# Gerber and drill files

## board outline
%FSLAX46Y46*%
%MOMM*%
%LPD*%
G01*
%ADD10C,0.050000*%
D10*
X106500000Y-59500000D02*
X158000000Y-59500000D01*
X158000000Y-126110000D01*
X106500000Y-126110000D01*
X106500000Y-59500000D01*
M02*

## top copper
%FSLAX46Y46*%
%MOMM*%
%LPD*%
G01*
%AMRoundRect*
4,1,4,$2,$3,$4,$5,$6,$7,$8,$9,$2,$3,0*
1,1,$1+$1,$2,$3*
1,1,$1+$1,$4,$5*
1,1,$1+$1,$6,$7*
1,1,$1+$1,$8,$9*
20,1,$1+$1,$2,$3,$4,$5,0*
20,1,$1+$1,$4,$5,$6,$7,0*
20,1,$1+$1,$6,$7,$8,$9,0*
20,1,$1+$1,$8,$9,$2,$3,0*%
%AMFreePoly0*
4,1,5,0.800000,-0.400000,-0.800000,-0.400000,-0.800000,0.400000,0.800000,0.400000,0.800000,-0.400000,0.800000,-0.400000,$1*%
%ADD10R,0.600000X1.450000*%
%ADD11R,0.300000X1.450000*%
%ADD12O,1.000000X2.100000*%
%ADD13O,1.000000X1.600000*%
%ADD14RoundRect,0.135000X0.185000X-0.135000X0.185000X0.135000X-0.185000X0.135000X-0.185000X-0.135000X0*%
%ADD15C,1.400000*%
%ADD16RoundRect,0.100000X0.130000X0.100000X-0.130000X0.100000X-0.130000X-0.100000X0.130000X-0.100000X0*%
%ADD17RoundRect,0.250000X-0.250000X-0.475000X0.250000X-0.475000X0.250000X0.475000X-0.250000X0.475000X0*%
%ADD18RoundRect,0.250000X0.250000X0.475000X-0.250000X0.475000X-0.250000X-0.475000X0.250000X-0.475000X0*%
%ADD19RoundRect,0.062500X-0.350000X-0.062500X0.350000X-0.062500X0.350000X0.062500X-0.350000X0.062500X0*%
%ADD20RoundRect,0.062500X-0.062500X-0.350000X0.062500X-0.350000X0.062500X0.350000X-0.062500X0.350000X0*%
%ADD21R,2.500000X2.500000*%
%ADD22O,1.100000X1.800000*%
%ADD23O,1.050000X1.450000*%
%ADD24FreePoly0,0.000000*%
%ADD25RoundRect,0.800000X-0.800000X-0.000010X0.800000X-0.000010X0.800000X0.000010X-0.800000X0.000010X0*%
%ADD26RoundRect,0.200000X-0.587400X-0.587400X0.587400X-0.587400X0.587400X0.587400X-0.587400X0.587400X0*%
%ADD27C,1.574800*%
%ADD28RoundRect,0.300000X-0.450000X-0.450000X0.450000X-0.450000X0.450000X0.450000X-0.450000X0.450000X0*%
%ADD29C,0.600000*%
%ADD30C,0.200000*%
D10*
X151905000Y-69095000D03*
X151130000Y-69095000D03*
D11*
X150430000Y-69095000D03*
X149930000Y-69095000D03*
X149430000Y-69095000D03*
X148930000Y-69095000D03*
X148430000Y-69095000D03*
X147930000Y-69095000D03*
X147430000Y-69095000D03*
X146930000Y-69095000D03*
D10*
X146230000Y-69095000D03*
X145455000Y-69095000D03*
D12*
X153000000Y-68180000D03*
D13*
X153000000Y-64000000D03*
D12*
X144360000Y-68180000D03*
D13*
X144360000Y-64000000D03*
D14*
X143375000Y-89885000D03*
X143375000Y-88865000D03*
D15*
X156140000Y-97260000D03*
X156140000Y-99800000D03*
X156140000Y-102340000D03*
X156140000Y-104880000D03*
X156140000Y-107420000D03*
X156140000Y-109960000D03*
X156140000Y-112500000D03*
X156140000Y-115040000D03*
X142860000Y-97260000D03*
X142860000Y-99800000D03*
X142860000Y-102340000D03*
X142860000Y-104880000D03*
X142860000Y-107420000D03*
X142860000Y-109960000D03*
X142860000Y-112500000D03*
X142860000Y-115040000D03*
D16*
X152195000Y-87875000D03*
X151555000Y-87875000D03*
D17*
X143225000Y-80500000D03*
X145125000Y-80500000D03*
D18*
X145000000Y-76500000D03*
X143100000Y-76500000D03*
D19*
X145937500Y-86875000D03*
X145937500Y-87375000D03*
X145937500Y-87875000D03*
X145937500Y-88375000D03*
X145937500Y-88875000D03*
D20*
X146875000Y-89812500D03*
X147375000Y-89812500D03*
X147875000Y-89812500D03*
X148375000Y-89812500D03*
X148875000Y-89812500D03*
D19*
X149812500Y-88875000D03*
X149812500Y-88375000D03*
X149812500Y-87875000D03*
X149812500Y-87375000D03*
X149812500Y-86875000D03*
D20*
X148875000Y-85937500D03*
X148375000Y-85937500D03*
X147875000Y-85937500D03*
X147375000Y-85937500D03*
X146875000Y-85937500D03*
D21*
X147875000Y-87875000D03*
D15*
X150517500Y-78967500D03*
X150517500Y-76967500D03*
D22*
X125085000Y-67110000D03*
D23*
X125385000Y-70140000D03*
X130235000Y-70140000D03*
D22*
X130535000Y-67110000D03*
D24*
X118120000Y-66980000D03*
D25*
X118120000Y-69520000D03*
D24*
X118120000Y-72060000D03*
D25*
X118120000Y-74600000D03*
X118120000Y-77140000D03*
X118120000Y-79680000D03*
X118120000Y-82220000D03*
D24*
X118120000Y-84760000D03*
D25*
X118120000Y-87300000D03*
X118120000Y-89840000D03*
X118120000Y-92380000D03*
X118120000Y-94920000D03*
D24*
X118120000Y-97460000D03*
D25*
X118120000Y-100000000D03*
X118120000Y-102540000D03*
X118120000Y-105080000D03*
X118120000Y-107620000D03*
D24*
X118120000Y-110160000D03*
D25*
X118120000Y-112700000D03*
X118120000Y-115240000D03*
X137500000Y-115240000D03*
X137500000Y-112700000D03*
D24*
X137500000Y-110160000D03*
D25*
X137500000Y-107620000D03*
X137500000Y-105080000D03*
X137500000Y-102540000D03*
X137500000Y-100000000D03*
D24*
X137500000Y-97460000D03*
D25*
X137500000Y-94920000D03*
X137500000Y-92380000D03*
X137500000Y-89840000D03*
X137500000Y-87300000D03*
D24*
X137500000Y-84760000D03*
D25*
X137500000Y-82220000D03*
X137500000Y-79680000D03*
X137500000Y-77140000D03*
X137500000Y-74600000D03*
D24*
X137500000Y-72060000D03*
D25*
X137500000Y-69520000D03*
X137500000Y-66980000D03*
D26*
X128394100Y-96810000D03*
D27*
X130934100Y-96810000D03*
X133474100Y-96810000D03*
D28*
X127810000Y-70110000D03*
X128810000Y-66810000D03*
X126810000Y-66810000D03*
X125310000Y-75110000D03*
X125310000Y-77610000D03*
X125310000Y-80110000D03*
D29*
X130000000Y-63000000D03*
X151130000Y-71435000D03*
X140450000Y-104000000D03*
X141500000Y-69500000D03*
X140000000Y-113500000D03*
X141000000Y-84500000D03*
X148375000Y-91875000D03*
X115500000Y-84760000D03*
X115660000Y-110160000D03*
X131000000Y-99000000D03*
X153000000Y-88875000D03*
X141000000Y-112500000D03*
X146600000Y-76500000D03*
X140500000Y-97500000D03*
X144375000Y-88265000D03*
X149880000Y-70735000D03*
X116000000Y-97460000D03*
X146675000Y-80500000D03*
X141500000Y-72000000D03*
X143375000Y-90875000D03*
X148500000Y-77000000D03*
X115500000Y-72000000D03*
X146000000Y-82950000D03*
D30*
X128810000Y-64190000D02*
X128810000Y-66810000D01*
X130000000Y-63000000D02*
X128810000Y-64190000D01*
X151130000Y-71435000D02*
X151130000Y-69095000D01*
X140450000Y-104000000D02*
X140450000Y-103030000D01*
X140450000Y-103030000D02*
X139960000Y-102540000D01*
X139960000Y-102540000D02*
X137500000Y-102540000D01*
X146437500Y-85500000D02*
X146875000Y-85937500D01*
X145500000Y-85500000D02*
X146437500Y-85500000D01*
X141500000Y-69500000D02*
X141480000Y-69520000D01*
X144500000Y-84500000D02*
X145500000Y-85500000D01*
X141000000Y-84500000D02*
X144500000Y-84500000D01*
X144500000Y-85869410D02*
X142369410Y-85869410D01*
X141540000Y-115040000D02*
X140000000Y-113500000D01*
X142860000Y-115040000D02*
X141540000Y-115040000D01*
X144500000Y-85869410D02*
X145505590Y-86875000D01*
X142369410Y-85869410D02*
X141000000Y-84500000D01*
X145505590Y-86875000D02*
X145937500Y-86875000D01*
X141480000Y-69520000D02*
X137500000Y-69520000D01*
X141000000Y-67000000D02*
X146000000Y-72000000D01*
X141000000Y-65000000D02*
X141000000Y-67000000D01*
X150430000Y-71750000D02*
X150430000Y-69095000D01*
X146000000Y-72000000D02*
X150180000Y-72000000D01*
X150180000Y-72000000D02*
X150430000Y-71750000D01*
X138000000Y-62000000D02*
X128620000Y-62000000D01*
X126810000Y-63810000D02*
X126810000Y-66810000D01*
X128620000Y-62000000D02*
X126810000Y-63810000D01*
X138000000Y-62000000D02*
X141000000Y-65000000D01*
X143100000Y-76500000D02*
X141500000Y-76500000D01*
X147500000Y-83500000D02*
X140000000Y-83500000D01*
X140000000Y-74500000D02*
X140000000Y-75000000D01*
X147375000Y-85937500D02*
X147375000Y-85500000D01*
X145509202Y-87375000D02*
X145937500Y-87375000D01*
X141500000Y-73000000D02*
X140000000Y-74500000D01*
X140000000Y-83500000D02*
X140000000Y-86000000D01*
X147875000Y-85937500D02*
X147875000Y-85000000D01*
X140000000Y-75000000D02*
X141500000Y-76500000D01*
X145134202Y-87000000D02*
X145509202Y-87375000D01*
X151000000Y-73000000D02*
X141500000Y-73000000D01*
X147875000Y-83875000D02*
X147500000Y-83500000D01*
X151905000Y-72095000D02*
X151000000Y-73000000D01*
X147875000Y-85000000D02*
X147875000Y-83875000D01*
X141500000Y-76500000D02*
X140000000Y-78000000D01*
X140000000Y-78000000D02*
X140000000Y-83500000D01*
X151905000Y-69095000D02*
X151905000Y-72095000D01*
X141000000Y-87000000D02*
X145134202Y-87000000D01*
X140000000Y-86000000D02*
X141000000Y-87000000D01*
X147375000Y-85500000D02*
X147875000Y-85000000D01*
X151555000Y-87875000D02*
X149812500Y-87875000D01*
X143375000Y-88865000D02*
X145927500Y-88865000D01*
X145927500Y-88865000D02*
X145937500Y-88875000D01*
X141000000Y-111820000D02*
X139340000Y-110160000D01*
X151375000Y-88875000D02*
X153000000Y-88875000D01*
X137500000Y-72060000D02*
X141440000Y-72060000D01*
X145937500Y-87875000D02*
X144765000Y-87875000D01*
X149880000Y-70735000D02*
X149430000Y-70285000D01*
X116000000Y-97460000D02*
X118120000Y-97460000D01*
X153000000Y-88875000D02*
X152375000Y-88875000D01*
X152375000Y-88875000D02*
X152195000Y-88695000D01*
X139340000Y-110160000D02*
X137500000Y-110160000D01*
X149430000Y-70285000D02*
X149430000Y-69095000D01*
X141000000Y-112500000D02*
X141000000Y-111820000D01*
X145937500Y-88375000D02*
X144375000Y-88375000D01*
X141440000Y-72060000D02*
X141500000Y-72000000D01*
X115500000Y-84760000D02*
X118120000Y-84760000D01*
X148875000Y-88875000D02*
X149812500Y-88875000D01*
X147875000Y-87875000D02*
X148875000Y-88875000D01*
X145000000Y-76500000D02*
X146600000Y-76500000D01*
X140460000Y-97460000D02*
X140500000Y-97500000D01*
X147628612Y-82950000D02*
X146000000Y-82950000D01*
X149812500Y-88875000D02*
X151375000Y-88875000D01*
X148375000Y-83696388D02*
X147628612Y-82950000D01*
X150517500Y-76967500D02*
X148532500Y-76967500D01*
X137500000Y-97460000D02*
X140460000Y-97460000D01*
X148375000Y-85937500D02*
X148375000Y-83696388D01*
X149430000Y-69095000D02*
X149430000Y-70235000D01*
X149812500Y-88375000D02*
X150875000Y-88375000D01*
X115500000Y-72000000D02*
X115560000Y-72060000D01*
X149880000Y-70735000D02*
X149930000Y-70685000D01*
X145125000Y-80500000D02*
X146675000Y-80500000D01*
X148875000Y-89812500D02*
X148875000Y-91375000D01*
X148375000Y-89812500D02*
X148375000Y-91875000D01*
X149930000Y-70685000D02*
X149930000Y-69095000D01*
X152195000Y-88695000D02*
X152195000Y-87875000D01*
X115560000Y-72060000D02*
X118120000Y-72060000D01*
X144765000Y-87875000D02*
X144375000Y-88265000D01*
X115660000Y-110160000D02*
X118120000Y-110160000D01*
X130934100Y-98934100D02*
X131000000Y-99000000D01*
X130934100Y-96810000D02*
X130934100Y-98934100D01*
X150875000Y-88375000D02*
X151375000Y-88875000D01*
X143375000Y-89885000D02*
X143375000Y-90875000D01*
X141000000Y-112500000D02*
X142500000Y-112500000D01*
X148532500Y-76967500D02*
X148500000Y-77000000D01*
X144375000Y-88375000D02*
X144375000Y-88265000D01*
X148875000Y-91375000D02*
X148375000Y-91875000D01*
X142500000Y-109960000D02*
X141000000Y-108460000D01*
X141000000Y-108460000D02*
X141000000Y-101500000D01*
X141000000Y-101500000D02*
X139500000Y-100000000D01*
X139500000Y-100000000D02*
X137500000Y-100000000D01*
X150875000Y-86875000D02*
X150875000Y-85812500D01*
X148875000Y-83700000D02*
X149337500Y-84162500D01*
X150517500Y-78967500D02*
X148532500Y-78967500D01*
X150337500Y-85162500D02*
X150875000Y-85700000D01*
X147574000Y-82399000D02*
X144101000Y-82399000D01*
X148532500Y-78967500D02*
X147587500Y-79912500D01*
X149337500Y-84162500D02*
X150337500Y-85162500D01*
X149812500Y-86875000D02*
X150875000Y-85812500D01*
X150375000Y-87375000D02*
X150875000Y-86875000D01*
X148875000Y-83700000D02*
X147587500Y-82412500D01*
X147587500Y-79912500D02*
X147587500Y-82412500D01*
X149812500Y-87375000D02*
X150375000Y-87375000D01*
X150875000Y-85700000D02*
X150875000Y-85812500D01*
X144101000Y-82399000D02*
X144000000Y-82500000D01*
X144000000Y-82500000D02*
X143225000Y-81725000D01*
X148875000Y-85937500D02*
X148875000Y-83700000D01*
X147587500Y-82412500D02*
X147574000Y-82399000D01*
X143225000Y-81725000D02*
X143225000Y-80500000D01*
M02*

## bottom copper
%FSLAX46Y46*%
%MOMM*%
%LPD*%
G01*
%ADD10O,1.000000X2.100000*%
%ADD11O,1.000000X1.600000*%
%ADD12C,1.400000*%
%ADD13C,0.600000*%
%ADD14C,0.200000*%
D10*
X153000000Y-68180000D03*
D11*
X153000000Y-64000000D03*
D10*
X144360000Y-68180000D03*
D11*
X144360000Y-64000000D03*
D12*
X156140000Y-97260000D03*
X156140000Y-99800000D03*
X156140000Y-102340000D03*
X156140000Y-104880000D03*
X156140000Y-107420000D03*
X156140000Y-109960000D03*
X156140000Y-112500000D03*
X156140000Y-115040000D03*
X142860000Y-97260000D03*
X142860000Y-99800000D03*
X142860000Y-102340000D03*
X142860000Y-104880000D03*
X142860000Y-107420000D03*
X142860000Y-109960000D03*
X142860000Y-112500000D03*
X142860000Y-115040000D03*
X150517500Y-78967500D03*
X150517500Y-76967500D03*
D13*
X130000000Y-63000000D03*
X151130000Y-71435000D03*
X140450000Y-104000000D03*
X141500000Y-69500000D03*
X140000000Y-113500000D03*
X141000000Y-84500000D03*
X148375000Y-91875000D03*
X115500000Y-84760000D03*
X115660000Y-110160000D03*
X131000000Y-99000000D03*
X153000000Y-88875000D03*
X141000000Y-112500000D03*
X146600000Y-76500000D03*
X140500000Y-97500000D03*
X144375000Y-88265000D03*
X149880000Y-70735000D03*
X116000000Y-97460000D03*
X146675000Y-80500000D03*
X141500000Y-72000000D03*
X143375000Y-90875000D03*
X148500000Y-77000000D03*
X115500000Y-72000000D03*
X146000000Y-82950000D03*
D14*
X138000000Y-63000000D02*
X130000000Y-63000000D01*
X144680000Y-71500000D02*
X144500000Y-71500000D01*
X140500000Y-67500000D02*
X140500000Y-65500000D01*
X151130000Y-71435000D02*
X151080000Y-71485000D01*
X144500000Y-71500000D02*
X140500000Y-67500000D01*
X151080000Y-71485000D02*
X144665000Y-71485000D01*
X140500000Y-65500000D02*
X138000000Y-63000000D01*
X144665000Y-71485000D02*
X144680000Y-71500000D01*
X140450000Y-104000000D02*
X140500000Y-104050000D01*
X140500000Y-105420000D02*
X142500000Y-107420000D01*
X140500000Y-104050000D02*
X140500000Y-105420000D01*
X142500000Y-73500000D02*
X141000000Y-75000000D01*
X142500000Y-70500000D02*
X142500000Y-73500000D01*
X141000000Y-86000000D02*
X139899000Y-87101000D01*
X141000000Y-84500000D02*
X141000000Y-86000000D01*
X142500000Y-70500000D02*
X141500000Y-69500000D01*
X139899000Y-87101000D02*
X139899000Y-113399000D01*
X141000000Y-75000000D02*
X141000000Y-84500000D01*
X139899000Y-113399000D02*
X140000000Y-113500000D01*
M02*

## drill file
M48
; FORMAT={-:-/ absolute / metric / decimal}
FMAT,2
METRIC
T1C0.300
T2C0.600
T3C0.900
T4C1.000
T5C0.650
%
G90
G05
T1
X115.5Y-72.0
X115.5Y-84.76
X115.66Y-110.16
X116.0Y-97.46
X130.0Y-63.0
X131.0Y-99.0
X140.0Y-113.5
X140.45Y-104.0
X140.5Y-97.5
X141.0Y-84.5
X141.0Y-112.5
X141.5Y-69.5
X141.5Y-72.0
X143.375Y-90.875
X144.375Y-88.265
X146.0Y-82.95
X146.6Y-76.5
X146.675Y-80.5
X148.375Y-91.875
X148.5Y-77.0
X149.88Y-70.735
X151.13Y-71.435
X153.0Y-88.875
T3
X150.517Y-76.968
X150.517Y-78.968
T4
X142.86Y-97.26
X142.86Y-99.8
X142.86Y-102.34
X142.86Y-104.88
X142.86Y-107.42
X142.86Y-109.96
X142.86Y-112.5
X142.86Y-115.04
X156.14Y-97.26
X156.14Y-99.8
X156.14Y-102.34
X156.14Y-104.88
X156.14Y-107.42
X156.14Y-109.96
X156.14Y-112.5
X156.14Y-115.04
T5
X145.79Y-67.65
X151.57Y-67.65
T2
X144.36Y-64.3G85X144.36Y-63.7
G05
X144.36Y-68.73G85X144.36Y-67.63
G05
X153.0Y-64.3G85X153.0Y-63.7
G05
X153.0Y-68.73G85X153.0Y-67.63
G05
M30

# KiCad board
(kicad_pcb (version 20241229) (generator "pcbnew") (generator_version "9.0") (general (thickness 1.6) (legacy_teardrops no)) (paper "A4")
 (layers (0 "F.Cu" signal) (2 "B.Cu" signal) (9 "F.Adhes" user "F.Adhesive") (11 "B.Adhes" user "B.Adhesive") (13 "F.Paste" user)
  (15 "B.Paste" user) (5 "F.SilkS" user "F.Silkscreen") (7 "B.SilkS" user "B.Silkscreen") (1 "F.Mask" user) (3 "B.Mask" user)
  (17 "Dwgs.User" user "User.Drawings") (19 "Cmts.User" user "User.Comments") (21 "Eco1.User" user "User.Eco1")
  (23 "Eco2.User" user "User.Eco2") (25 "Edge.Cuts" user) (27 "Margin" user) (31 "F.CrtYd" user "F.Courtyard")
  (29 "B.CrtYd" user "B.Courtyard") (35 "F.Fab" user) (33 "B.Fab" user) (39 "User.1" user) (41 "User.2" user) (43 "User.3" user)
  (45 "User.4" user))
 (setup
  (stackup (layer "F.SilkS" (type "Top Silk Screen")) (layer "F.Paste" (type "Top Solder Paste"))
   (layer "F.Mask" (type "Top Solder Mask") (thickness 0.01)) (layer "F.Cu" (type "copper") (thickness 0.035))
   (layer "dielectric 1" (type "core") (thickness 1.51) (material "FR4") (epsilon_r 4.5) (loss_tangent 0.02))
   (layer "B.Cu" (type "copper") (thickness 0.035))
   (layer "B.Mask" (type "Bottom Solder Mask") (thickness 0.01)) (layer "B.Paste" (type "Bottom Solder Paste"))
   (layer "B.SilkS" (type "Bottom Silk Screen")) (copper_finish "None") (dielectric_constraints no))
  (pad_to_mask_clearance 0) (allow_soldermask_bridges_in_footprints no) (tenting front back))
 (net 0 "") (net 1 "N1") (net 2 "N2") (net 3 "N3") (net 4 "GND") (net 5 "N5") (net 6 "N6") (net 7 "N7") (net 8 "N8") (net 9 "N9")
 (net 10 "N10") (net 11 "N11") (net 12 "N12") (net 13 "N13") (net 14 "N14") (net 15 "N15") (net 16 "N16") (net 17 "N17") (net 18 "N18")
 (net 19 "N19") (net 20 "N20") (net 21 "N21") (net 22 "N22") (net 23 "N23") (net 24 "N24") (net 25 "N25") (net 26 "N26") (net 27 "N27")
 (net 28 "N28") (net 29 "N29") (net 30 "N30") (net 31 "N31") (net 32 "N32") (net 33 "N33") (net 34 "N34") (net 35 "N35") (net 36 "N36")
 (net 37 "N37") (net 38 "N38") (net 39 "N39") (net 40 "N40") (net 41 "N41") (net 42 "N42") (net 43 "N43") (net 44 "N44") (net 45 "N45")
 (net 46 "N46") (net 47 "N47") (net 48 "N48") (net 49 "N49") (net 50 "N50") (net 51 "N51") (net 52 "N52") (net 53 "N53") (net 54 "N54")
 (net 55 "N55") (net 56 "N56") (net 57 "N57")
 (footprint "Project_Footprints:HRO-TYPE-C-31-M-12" (layer "F.Cu") (at 148.68 61.4 180)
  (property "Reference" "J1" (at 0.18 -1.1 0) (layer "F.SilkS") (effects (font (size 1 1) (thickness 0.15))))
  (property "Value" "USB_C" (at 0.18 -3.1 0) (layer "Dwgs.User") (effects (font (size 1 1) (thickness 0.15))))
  (pad "" np_thru_hole circle (at -2.89 -6.25 180) (size 0.65 0.65) (drill 0.65) (layers "*.Cu" "*.Mask"))
  (pad "" np_thru_hole circle (at 2.89 -6.25 180) (size 0.65 0.65) (drill 0.65) (layers "*.Cu" "*.Mask"))
  (pad "1" smd rect (at -3.225 -7.695 180) (size 0.6 1.45) (layers "F.Cu" "F.Mask" "F.Paste") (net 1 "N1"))
  (pad "2" smd rect (at -2.45 -7.695 180) (size 0.6 1.45) (layers "F.Cu" "F.Mask" "F.Paste") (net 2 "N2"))
  (pad "3" smd rect (at -1.75 -7.695 180) (size 0.3 1.45) (layers "F.Cu" "F.Mask" "F.Paste") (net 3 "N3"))
  (pad "4" smd rect (at -1.25 -7.695 180) (size 0.3 1.45) (layers "F.Cu" "F.Mask" "F.Paste") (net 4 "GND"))
  (pad "5" smd rect (at -0.75 -7.695 180) (size 0.3 1.45) (layers "F.Cu" "F.Mask" "F.Paste") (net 4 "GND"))
  (pad "6" smd rect (at -0.25 -7.695 180) (size 0.3 1.45) (layers "F.Cu" "F.Mask" "F.Paste"))
  (pad "7" smd rect (at 0.25 -7.695 180) (size 0.3 1.45) (layers "F.Cu" "F.Mask" "F.Paste"))
  (pad "8" smd rect (at 0.75 -7.695 180) (size 0.3 1.45) (layers "F.Cu" "F.Mask" "F.Paste"))
  (pad "9" smd rect (at 1.25 -7.695 180) (size 0.3 1.45) (layers "F.Cu" "F.Mask" "F.Paste"))
  (pad "10" smd rect (at 1.75 -7.695 180) (size 0.3 1.45) (layers "F.Cu" "F.Mask" "F.Paste"))
  (pad "11" smd rect (at 2.45 -7.695 180) (size 0.6 1.45) (layers "F.Cu" "F.Mask" "F.Paste"))
  (pad "12" smd rect (at 3.225 -7.695 180) (size 0.6 1.45) (layers "F.Cu" "F.Mask" "F.Paste"))
  (pad "13" thru_hole oval (at -4.32 -6.78 180) (size 1 2.1) (drill oval 0.6 1.7) (layers "*.Cu" "B.Mask") (remove_unused_layers no))
  (pad "13" thru_hole oval (at -4.32 -2.6 180) (size 1 1.6) (drill oval 0.6 1.2) (layers "*.Cu" "B.Mask") (remove_unused_layers no))
  (pad "13" thru_hole oval (at 4.32 -6.78 180) (size 1 2.1) (drill oval 0.6 1.7) (layers "*.Cu" "B.Mask") (remove_unused_layers no))
  (pad "13" thru_hole oval (at 4.32 -2.6 180) (size 1 1.6) (drill oval 0.6 1.2) (layers "*.Cu" "B.Mask") (remove_unused_layers no)))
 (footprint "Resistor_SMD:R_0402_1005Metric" (layer "F.Cu") (at 143.375 89.375 90)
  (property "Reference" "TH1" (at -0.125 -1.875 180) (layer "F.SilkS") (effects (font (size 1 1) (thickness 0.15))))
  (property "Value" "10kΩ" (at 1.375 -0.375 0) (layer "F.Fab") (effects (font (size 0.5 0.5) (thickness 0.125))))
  (pad "1" smd roundrect (at -0.51 0 90) (size 0.54 0.64) (layers "F.Cu" "F.Mask" "F.Paste") (roundrect_rratio 0.25) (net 4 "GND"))
  (pad "2" smd roundrect (at 0.51 0 90) (size 0.54 0.64) (layers "F.Cu" "F.Mask" "F.Paste") (roundrect_rratio 0.25) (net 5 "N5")))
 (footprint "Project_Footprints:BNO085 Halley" (layer "F.Cu") (at 156.14 97.26 -90)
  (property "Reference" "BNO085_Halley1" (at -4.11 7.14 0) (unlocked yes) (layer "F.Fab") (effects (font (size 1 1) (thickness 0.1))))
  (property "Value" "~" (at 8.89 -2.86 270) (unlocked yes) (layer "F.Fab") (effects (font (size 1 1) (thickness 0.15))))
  (pad "1" thru_hole circle (at 0 0 270) (size 1.4 1.4) (drill 1) (layers "*.Cu" "*.Mask") (remove_unused_layers no) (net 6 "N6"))
  (pad "2" thru_hole circle (at 2.54 0 270) (size 1.4 1.4) (drill 1) (layers "*.Cu" "*.Mask") (remove_unused_layers no) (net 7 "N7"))
  (pad "3" thru_hole circle (at 5.08 0 270) (size 1.4 1.4) (drill 1) (layers "*.Cu" "*.Mask") (remove_unused_layers no) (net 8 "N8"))
  (pad "4" thru_hole circle (at 7.62 0 270) (size 1.4 1.4) (drill 1) (layers "*.Cu" "*.Mask") (remove_unused_layers no) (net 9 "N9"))
  (pad "5" thru_hole circle (at 10.16 0 270) (size 1.4 1.4) (drill 1) (layers "*.Cu" "*.Mask") (remove_unused_layers no) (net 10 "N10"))
  (pad "6" thru_hole circle (at 12.7 0 270) (size 1.4 1.4) (drill 1) (layers "*.Cu" "*.Mask") (remove_unused_layers no) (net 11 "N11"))
  (pad "7" thru_hole circle (at 15.24 0 270) (size 1.4 1.4) (drill 1) (layers "*.Cu" "*.Mask") (remove_unused_layers no) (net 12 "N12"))
  (pad "8" thru_hole circle (at 17.78 0 270) (size 1.4 1.4) (drill 1) (layers "*.Cu" "*.Mask") (remove_unused_layers no) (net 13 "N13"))
  (pad "9" thru_hole circle (at 0 13.28 270) (size 1.4 1.4) (drill 1) (layers "*.Cu" "*.Mask") (remove_unused_layers no))
  (pad "10" thru_hole circle (at 2.54 13.28 270) (size 1.4 1.4) (drill 1) (layers "*.Cu" "*.Mask") (remove_unused_layers no))
  (pad "11" thru_hole circle (at 5.08 13.28 270) (size 1.4 1.4) (drill 1) (layers "*.Cu" "*.Mask") (remove_unused_layers no))
  (pad "12" thru_hole circle (at 7.62 13.28 270) (size 1.4 1.4) (drill 1) (layers "*.Cu" "*.Mask") (remove_unused_layers no))
  (pad "13" thru_hole circle (at 10.16 13.28 270) (size 1.4 1.4) (drill 1) (layers "*.Cu" "*.Mask") (remove_unused_layers no) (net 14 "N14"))
  (pad "14" thru_hole circle (at 12.7 13.28 270) (size 1.4 1.4) (drill 1) (layers "*.Cu" "*.Mask") (remove_unused_layers no) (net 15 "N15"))
  (pad "15" thru_hole circle (at 15.24 13.28 270) (size 1.4 1.4) (drill 1) (layers "*.Cu" "*.Mask") (remove_unused_layers no) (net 4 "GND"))
  (pad "16" thru_hole circle (at 17.78 13.28 270) (size 1.4 1.4) (drill 1) (layers "*.Cu" "*.Mask") (remove_unused_layers no) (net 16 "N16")))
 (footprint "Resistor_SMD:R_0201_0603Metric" (layer "F.Cu") (at 151.875 87.875 180)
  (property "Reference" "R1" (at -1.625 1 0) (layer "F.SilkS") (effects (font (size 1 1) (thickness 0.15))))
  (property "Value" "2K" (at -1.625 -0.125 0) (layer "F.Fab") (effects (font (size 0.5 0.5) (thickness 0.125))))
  (pad "" smd roundrect (at -0.345 0 180) (size 0.318 0.36) (layers "F.Paste") (roundrect_rratio 0.25))
  (pad "" smd roundrect (at 0.345 0 180) (size 0.318 0.36) (layers "F.Paste") (roundrect_rratio 0.25))
  (pad "1" smd roundrect (at -0.32 0 180) (size 0.46 0.4) (layers "F.Cu" "F.Mask") (roundrect_rratio 0.25) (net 4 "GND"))
  (pad "2" smd roundrect (at 0.32 0 180) (size 0.46 0.4) (layers "F.Cu" "F.Mask") (roundrect_rratio 0.25) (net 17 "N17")))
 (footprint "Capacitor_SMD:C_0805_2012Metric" (layer "F.Cu") (at 144.175 80.5)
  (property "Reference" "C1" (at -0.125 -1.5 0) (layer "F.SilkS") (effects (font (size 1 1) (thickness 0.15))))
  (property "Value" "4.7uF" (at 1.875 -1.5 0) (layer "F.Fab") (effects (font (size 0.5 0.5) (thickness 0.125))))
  (pad "1" smd roundrect (at -0.95 0) (size 1 1.45) (layers "F.Cu" "F.Mask" "F.Paste") (roundrect_rratio 0.25) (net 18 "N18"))
  (pad "2" smd roundrect (at 0.95 0) (size 1 1.45) (layers "F.Cu" "F.Mask" "F.Paste") (roundrect_rratio 0.25) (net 4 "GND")))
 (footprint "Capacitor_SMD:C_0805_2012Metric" (layer "F.Cu") (at 144.05 76.5 180)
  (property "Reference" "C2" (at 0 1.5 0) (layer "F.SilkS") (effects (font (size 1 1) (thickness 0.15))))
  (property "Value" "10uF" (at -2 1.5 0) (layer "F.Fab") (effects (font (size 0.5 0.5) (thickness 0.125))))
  (pad "1" smd roundrect (at -0.95 0 180) (size 1 1.45) (layers "F.Cu" "F.Mask" "F.Paste") (roundrect_rratio 0.25) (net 4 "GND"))
  (pad "2" smd roundrect (at 0.95 0 180) (size 1 1.45) (layers "F.Cu" "F.Mask" "F.Paste") (roundrect_rratio 0.25) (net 1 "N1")))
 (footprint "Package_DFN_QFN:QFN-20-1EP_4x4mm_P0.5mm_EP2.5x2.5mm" (layer "F.Cu") (at 147.875 87.875)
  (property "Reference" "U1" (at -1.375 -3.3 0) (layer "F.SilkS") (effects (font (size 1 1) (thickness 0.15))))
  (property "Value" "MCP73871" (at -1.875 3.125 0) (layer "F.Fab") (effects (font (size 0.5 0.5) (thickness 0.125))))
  (pad "" smd roundrect (at -0.625 -0.625) (size 1.01 1.01) (layers "F.Paste") (roundrect_rratio 0.247525))
  (pad "" smd roundrect (at -0.625 0.625) (size 1.01 1.01) (layers "F.Paste") (roundrect_rratio 0.247525))
  (pad "" smd roundrect (at 0.625 -0.625) (size 1.01 1.01) (layers "F.Paste") (roundrect_rratio 0.247525))
  (pad "" smd roundrect (at 0.625 0.625) (size 1.01 1.01) (layers "F.Paste") (roundrect_rratio 0.247525))
  (pad "1" smd roundrect (at -1.9375 -1) (size 0.825 0.25) (layers "F.Cu" "F.Mask" "F.Paste") (roundrect_rratio 0.25) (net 16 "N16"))
  (pad "2" smd roundrect (at -1.9375 -0.5) (size 0.825 0.25) (layers "F.Cu" "F.Mask" "F.Paste") (roundrect_rratio 0.25) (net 1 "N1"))
  (pad "3" smd roundrect (at -1.9375 0) (size 0.825 0.25) (layers "F.Cu" "F.Mask" "F.Paste") (roundrect_rratio 0.25) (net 4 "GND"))
  (pad "4" smd roundrect (at -1.9375 0.5) (size 0.825 0.25) (layers "F.Cu" "F.Mask" "F.Paste") (roundrect_rratio 0.25) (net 4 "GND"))
  (pad "5" smd roundrect (at -1.9375 1) (size 0.825 0.25) (layers "F.Cu" "F.Mask" "F.Paste") (roundrect_rratio 0.25) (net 5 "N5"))
  (pad "6" smd roundrect (at -1 1.9375) (size 0.25 0.825) (layers "F.Cu" "F.Mask" "F.Paste") (roundrect_rratio 0.25) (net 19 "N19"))
  (pad "7" smd roundrect (at -0.5 1.9375) (size 0.25 0.825) (layers "F.Cu" "F.Mask" "F.Paste") (roundrect_rratio 0.25) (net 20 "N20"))
  (pad "8" smd roundrect (at 0 1.9375) (size 0.25 0.825) (layers "F.Cu" "F.Mask" "F.Paste") (roundrect_rratio 0.25) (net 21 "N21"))
  (pad "9" smd roundrect (at 0.5 1.9375) (size 0.25 0.825) (layers "F.Cu" "F.Mask" "F.Paste") (roundrect_rratio 0.25) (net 4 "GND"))
  (pad "10" smd roundrect (at 1 1.9375) (size 0.25 0.825) (layers "F.Cu" "F.Mask" "F.Paste") (roundrect_rratio 0.25) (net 4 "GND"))
  (pad "11" smd roundrect (at 1.9375 1) (size 0.825 0.25) (layers "F.Cu" "F.Mask" "F.Paste") (roundrect_rratio 0.25) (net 4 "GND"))
  (pad "12" smd roundrect (at 1.9375 0.5) (size 0.825 0.25) (layers "F.Cu" "F.Mask" "F.Paste") (roundrect_rratio 0.25) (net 4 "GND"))
  (pad "13" smd roundrect (at 1.9375 0) (size 0.825 0.25) (layers "F.Cu" "F.Mask" "F.Paste") (roundrect_rratio 0.25) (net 17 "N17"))
  (pad "14" smd roundrect (at 1.9375 -0.5) (size 0.825 0.25) (layers "F.Cu" "F.Mask" "F.Paste") (roundrect_rratio 0.25) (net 18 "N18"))
  (pad "15" smd roundrect (at 1.9375 -1) (size 0.825 0.25) (layers "F.Cu" "F.Mask" "F.Paste") (roundrect_rratio 0.25) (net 18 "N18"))
  (pad "16" smd roundrect (at 1 -1.9375) (size 0.25 0.825) (layers "F.Cu" "F.Mask" "F.Paste") (roundrect_rratio 0.25) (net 18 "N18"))
  (pad "17" smd roundrect (at 0.5 -1.9375) (size 0.25 0.825) (layers "F.Cu" "F.Mask" "F.Paste") (roundrect_rratio 0.25) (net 4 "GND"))
  (pad "18" smd roundrect (at 0 -1.9375) (size 0.25 0.825) (layers "F.Cu" "F.Mask" "F.Paste") (roundrect_rratio 0.25) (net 1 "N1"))
  (pad "19" smd roundrect (at -0.5 -1.9375) (size 0.25 0.825) (layers "F.Cu" "F.Mask" "F.Paste") (roundrect_rratio 0.25) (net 1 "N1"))
  (pad "20" smd roundrect (at -1 -1.9375) (size 0.25 0.825) (layers "F.Cu" "F.Mask" "F.Paste") (roundrect_rratio 0.25) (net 16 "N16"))
  (pad "21" smd rect (at 0 0) (size 2.5 2.5) (layers "F.Cu" "F.Mask") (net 4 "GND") (zone_connect 2)))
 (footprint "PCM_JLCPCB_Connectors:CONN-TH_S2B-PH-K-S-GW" (layer "F.Cu") (at 150.5175 77.9675 -90)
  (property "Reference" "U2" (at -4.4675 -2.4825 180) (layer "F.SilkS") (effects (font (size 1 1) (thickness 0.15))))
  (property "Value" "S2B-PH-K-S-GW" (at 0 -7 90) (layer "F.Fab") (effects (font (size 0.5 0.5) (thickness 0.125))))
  (pad "1" thru_hole circle (at 1 0 270) (size 1.4 1.4) (drill 0.900024) (layers "*.Cu" "*.Mask") (remove_unused_layers no) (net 18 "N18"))
  (pad "2" thru_hole circle (at -1 0 270) (size 1.4 1.4) (drill 0.900024) (layers "*.Cu" "*.Mask") (remove_unused_layers no) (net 4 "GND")))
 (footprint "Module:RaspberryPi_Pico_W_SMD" (layer "F.Cu") (at 127.81 91.11)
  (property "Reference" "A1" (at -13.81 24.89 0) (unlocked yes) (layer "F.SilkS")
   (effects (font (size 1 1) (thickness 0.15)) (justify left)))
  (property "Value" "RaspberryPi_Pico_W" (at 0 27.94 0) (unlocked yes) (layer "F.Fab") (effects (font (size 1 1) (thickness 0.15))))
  (pad "" smd rect (at -8.89 -24.13) (size 3.8 2.2) (drill (offset -0.8 0)) (layers "F.Paste"))
  (pad "" smd rect (at -8.89 -21.59) (size 3.8 2.2) (drill (offset -0.8 0)) (layers "F.Paste"))
  (pad "" smd rect (at -8.89 -19.05) (size 3.8 2.2) (drill (offset -0.8 0)) (layers "F.Paste"))
  (pad "" smd rect (at -8.89 -16.51) (size 3.8 2.2) (drill (offset -0.8 0)) (layers "F.Paste"))
  (pad "" smd rect (at -8.89 -13.97) (size 3.8 2.2) (drill (offset -0.8 0)) (layers "F.Paste"))
  (pad "" smd rect (at -8.89 -11.43) (size 3.8 2.2) (drill (offset -0.8 0)) (layers "F.Paste"))
  (pad "" smd rect (at -8.89 -8.89) (size 3.8 2.2) (drill (offset -0.8 0)) (layers "F.Paste"))
  (pad "" smd rect (at -8.89 -6.35) (size 3.8 2.2) (drill (offset -0.8 0)) (layers "F.Paste"))
  (pad "" smd rect (at -8.89 -3.81) (size 3.8 2.2) (drill (offset -0.8 0)) (layers "F.Paste"))
  (pad "" smd rect (at -8.89 -1.27) (size 3.8 2.2) (drill (offset -0.8 0)) (layers "F.Paste"))
  (pad "" smd rect (at -8.89 1.27) (size 3.8 2.2) (drill (offset -0.8 0)) (layers "F.Paste"))
  (pad "" smd rect (at -8.89 3.81) (size 3.8 2.2) (drill (offset -0.8 0)) (layers "F.Paste"))
  (pad "" smd rect (at -8.89 6.35) (size 3.8 2.2) (drill (offset -0.8 0)) (layers "F.Paste"))
  (pad "" smd rect (at -8.89 8.89) (size 3.8 2.2) (drill (offset -0.8 0)) (layers "F.Paste"))
  (pad "" smd rect (at -8.89 11.43) (size 3.8 2.2) (drill (offset -0.8 0)) (layers "F.Paste"))
  (pad "" smd rect (at -8.89 13.97) (size 3.8 2.2) (drill (offset -0.8 0)) (layers "F.Paste"))
  (pad "" smd rect (at -8.89 16.51) (size 3.8 2.2) (drill (offset -0.8 0)) (layers "F.Paste"))
  (pad "" smd rect (at -8.89 19.05) (size 3.8 2.2) (drill (offset -0.8 0)) (layers "F.Paste"))
  (pad "" smd rect (at -8.89 21.59) (size 3.8 2.2) (drill (offset -0.8 0)) (layers "F.Paste"))
  (pad "" smd rect (at -8.89 24.13) (size 3.8 2.2) (drill (offset -0.8 0)) (layers "F.Paste"))
  (pad "" smd oval (at -2.725 -24) (size 1.1 1.8) (layers "F.Cu" "F.Mask" "F.Paste"))
  (pad "" smd oval (at -2.425 -20.97) (size 1.05 1.45) (layers "F.Cu" "F.Mask" "F.Paste"))
  (pad "" smd oval (at 2.425 -20.97) (size 1.05 1.45) (layers "F.Cu" "F.Mask" "F.Paste"))
  (pad "" smd oval (at 2.725 -24) (size 1.1 1.8) (layers "F.Cu" "F.Mask" "F.Paste"))
  (pad "" smd rect (at 8.89 -24.13) (size 3.8 2.2) (drill (offset 0.8 0)) (layers "F.Paste"))
  (pad "" smd rect (at 8.89 -21.59) (size 3.8 2.2) (drill (offset 0.8 0)) (layers "F.Paste"))
  (pad "" smd rect (at 8.89 -19.05) (size 3.8 2.2) (drill (offset 0.8 0)) (layers "F.Paste"))
  (pad "" smd rect (at 8.89 -16.51) (size 3.8 2.2) (drill (offset 0.8 0)) (layers "F.Paste"))
  (pad "" smd rect (at 8.89 -13.97) (size 3.8 2.2) (drill (offset 0.8 0)) (layers "F.Paste"))
  (pad "" smd rect (at 8.89 -11.43) (size 3.8 2.2) (drill (offset 0.8 0)) (layers "F.Paste"))
  (pad "" smd rect (at 8.89 -8.89) (size 3.8 2.2) (drill (offset 0.8 0)) (layers "F.Paste"))
  (pad "" smd rect (at 8.89 -6.35) (size 3.8 2.2) (drill (offset 0.8 0)) (layers "F.Paste"))
  (pad "" smd rect (at 8.89 -3.81) (size 3.8 2.2) (drill (offset 0.8 0)) (layers "F.Paste"))
  (pad "" smd rect (at 8.89 -1.27) (size 3.8 2.2) (drill (offset 0.8 0)) (layers "F.Paste"))
  (pad "" smd rect (at 8.89 1.27) (size 3.8 2.2) (drill (offset 0.8 0)) (layers "F.Paste"))
  (pad "" smd rect (at 8.89 3.81) (size 3.8 2.2) (drill (offset 0.8 0)) (layers "F.Paste"))
  (pad "" smd rect (at 8.89 6.35) (size 3.8 2.2) (drill (offset 0.8 0)) (layers "F.Paste"))
  (pad "" smd rect (at 8.89 8.89) (size 3.8 2.2) (drill (offset 0.8 0)) (layers "F.Paste"))
  (pad "" smd rect (at 8.89 11.43) (size 3.8 2.2) (drill (offset 0.8 0)) (layers "F.Paste"))
  (pad "" smd rect (at 8.89 13.97) (size 3.8 2.2) (drill (offset 0.8 0)) (layers "F.Paste"))
  (pad "" smd rect (at 8.89 16.51) (size 3.8 2.2) (drill (offset 0.8 0)) (layers "F.Paste"))
  (pad "" smd rect (at 8.89 19.05) (size 3.8 2.2) (drill (offset 0.8 0)) (layers "F.Paste"))
  (pad "" smd rect (at 8.89 21.59) (size 3.8 2.2) (drill (offset 0.8 0)) (layers "F.Paste"))
  (pad "" smd rect (at 8.89 24.13) (size 3.8 2.2) (drill (offset 0.8 0)) (layers "F.Paste"))
  (pad "1" smd custom (at -9.69 -24.13) (size 1.6 0.8) (layers "F.Cu" "F.Mask") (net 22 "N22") (options (clearance outline) (anchor rect))
   (primitives))
  (pad "2" smd roundrect (at -9.69 -21.59) (size 3.2 1.6) (layers "F.Cu" "F.Mask") (roundrect_rratio 0.5) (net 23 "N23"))
  (pad "3" smd custom (at -9.69 -19.05) (size 1.6 0.8) (layers "F.Cu" "F.Mask") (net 4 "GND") (options (clearance outline) (anchor rect))
   (primitives))
  (pad "4" smd roundrect (at -9.69 -16.51) (size 3.2 1.6) (layers "F.Cu" "F.Mask") (roundrect_rratio 0.5) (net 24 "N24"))
  (pad "5" smd roundrect (at -9.69 -13.97) (size 3.2 1.6) (layers "F.Cu" "F.Mask") (roundrect_rratio 0.5) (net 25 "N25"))
  (pad "6" smd roundrect (at -9.69 -11.43) (size 3.2 1.6) (layers "F.Cu" "F.Mask") (roundrect_rratio 0.5) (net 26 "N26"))
  (pad "7" smd roundrect (at -9.69 -8.89) (size 3.2 1.6) (layers "F.Cu" "F.Mask") (roundrect_rratio 0.5) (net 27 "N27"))
  (pad "8" smd custom (at -9.69 -6.35) (size 1.6 0.8) (layers "F.Cu" "F.Mask") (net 4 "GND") (options (clearance outline) (anchor rect))
   (primitives))
  (pad "9" smd roundrect (at -9.69 -3.81) (size 3.2 1.6) (layers "F.Cu" "F.Mask") (roundrect_rratio 0.5) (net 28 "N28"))
  (pad "10" smd roundrect (at -9.69 -1.27) (size 3.2 1.6) (layers "F.Cu" "F.Mask") (roundrect_rratio 0.5) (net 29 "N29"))
  (pad "11" smd roundrect (at -9.69 1.27) (size 3.2 1.6) (layers "F.Cu" "F.Mask") (roundrect_rratio 0.5) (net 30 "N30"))
  (pad "12" smd roundrect (at -9.69 3.81) (size 3.2 1.6) (layers "F.Cu" "F.Mask") (roundrect_rratio 0.5) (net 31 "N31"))
  (pad "13" smd custom (at -9.69 6.35) (size 1.6 0.8) (layers "F.Cu" "F.Mask") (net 4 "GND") (options (clearance outline) (anchor rect))
   (primitives))
  (pad "14" smd roundrect (at -9.69 8.89) (size 3.2 1.6) (layers "F.Cu" "F.Mask") (roundrect_rratio 0.5) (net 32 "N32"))
  (pad "15" smd roundrect (at -9.69 11.43) (size 3.2 1.6) (layers "F.Cu" "F.Mask") (roundrect_rratio 0.5) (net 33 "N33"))
  (pad "16" smd roundrect (at -9.69 13.97) (size 3.2 1.6) (layers "F.Cu" "F.Mask") (roundrect_rratio 0.5) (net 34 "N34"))
  (pad "17" smd roundrect (at -9.69 16.51) (size 3.2 1.6) (layers "F.Cu" "F.Mask") (roundrect_rratio 0.5) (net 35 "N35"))
  (pad "18" smd custom (at -9.69 19.05) (size 1.6 0.8) (layers "F.Cu" "F.Mask") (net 4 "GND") (options (clearance outline) (anchor rect))
   (primitives))
  (pad "19" smd roundrect (at -9.69 21.59) (size 3.2 1.6) (layers "F.Cu" "F.Mask") (roundrect_rratio 0.5) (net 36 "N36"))
  (pad "20" smd roundrect (at -9.69 24.13) (size 3.2 1.6) (layers "F.Cu" "F.Mask") (roundrect_rratio 0.5) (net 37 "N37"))
  (pad "21" smd roundrect (at 9.69 24.13) (size 3.2 1.6) (layers "F.Cu" "F.Mask") (roundrect_rratio 0.5) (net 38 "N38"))
  (pad "22" smd roundrect (at 9.69 21.59) (size 3.2 1.6) (layers "F.Cu" "F.Mask") (roundrect_rratio 0.5) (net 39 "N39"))
  (pad "23" smd custom (at 9.69 19.05) (size 1.6 0.8) (layers "F.Cu" "F.Mask") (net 4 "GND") (options (clearance outline) (anchor rect))
   (primitives))
  (pad "24" smd roundrect (at 9.69 16.51) (size 3.2 1.6) (layers "F.Cu" "F.Mask") (roundrect_rratio 0.5) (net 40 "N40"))
  (pad "25" smd roundrect (at 9.69 13.97) (size 3.2 1.6) (layers "F.Cu" "F.Mask") (roundrect_rratio 0.5) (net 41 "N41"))
  (pad "26" smd roundrect (at 9.69 11.43) (size 3.2 1.6) (layers "F.Cu" "F.Mask") (roundrect_rratio 0.5) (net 14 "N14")
   (padstack (mode front_inner_back)
    (layer "Inner" (shape roundrect) (size 3.2 1.6) (roundrect_rratio 0.5) (thermal_bridge_angle 45) (zone_connect -1))
    (layer "B.Cu" (shape roundrect) (size 3.2 1.6) (roundrect_rratio 0.5) (thermal_bridge_angle 45) (zone_connect -1))))
  (pad "27" smd roundrect (at 9.69 8.89) (size 3.2 1.6) (layers "F.Cu" "F.Mask") (roundrect_rratio 0.5) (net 15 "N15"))
  (pad "28" smd custom (at 9.69 6.35) (size 1.6 0.8) (layers "F.Cu" "F.Mask") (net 4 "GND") (options (clearance outline) (anchor rect))
   (primitives))
  (pad "29" smd roundrect (at 9.69 3.81) (size 3.2 1.6) (layers "F.Cu" "F.Mask") (roundrect_rratio 0.5) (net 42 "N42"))
  (pad "30" smd roundrect (at 9.69 1.27) (size 3.2 1.6) (layers "F.Cu" "F.Mask") (roundrect_rratio 0.5) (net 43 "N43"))
  (pad "31" smd roundrect (at 9.69 -1.27) (size 3.2 1.6) (layers "F.Cu" "F.Mask") (roundrect_rratio 0.5) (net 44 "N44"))
  (pad "32" smd roundrect (at 9.69 -3.81) (size 3.2 1.6) (layers "F.Cu" "F.Mask") (roundrect_rratio 0.5) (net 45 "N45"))
  (pad "33" smd custom (at 9.69 -6.35) (size 1.6 0.8) (layers "F.Cu" "F.Mask") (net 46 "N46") (options (clearance outline) (anchor rect))
   (primitives))
  (pad "34" smd roundrect (at 9.69 -8.89) (size 3.2 1.6) (layers "F.Cu" "F.Mask") (roundrect_rratio 0.5) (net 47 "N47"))
  (pad "35" smd roundrect (at 9.69 -11.43) (size 3.2 1.6) (layers "F.Cu" "F.Mask") (roundrect_rratio 0.5) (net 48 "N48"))
  (pad "36" smd roundrect (at 9.69 -13.97) (size 3.2 1.6) (layers "F.Cu" "F.Mask") (roundrect_rratio 0.5) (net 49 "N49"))
  (pad "37" smd roundrect (at 9.69 -16.51) (size 3.2 1.6) (layers "F.Cu" "F.Mask") (roundrect_rratio 0.5) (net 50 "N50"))
  (pad "38" smd custom (at 9.69 -19.05) (size 1.6 0.8) (layers "F.Cu" "F.Mask") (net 4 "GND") (options (clearance outline) (anchor rect))
   (primitives))
  (pad "39" smd roundrect (at 9.69 -21.59) (size 3.2 1.6) (layers "F.Cu" "F.Mask") (roundrect_rratio 0.5) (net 16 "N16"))
  (pad "40" smd roundrect (at 9.69 -24.13) (size 3.2 1.6) (layers "F.Cu" "F.Mask") (roundrect_rratio 0.5) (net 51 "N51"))
  (pad "D1" smd roundrect (at 0.5841 5.7) (size 1.5748 1.5748) (layers "F.Cu" "F.Mask" "F.Paste") (roundrect_rratio 0.127000254)
   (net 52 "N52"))
  (pad "D2" smd circle (at 3.1241 5.7) (size 1.5748 1.5748) (layers "F.Cu" "F.Mask" "F.Paste") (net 4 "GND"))
  (pad "D3" smd circle (at 5.6641 5.7) (size 1.5748 1.5748) (layers "F.Cu" "F.Mask" "F.Paste") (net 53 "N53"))
  (pad "TP1" smd roundrect (at 0 -21) (size 1.5 1.5) (layers "F.Cu" "F.Mask" "F.Paste") (roundrect_rratio 0.2) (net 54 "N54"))
  (pad "TP2" smd roundrect (at 1 -24.3) (size 1.5 1.5) (layers "F.Cu" "F.Mask" "F.Paste") (roundrect_rratio 0.2) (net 2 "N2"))
  (pad "TP3" smd roundrect (at -1 -24.3) (size 1.5 1.5) (layers "F.Cu" "F.Mask" "F.Paste") (roundrect_rratio 0.2) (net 3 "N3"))
  (pad "TP4" smd roundrect (at -2.5 -16) (size 1.5 1.5) (layers "F.Cu" "F.Mask" "F.Paste") (roundrect_rratio 0.2) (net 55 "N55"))
  (pad "TP5" smd roundrect (at -2.5 -13.5) (size 1.5 1.5) (layers "F.Cu" "F.Mask" "F.Paste") (roundrect_rratio 0.2) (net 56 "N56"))
  (pad "TP6" smd roundrect (at -2.5 -11) (size 1.5 1.5) (layers "F.Cu" "F.Mask" "F.Paste") (roundrect_rratio 0.2) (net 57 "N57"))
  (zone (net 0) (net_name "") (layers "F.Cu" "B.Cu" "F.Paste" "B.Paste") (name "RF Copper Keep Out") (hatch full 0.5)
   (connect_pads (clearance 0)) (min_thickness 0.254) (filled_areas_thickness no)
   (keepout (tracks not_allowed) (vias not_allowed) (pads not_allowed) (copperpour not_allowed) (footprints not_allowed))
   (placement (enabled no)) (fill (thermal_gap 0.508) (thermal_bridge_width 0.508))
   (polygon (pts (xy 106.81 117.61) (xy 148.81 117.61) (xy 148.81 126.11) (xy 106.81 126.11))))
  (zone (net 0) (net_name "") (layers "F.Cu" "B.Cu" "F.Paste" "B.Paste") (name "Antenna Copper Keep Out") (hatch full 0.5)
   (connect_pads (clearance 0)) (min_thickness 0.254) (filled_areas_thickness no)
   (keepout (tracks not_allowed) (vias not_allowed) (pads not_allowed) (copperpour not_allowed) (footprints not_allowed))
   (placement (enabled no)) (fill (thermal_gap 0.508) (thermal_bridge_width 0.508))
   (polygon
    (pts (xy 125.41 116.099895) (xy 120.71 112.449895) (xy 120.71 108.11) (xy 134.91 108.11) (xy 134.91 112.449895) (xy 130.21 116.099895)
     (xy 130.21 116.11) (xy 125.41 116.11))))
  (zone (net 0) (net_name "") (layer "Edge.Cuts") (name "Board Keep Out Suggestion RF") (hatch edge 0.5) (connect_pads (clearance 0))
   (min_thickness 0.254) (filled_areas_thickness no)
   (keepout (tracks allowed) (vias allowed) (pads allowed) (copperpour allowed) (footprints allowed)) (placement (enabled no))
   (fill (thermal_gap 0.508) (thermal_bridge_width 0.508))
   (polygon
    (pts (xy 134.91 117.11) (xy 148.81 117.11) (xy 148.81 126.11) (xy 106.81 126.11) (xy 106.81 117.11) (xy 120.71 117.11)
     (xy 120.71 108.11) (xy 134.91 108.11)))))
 (gr_rect (start 106.5 59.5) (end 158 126.11) (stroke (width 0.05) (type default)) (fill no) (layer "Edge.Cuts"))
 (segment (start 128.81 64.19) (end 128.81 66.81) (width 0.2) (layer "F.Cu") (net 2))
 (segment (start 130 63) (end 128.81 64.19) (width 0.2) (layer "F.Cu") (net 2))
 (segment (start 151.13 71.435) (end 151.13 69.095) (width 0.2) (layer "F.Cu") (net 2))
 (via (at 130 63) (size 0.6) (drill 0.3) (layers "F.Cu" "B.Cu") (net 2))
 (via (at 151.13 71.435) (size 0.6) (drill 0.3) (layers "F.Cu" "B.Cu") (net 2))
 (segment (start 138 63) (end 130 63) (width 0.2) (layer "B.Cu") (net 2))
 (segment (start 144.68 71.5) (end 144.5 71.5) (width 0.2) (layer "B.Cu") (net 2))
 (segment (start 140.5 67.5) (end 140.5 65.5) (width 0.2) (layer "B.Cu") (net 2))
 (segment (start 151.13 71.435) (end 151.08 71.485) (width 0.2) (layer "B.Cu") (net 2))
 (segment (start 144.5 71.5) (end 140.5 67.5) (width 0.2) (layer "B.Cu") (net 2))
 (segment (start 151.08 71.485) (end 144.665 71.485) (width 0.2) (layer "B.Cu") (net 2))
 (segment (start 140.5 65.5) (end 138 63) (width 0.2) (layer "B.Cu") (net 2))
 (segment (start 144.665 71.485) (end 144.68 71.5) (width 0.2) (layer "B.Cu") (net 2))
 (segment (start 140.45 104) (end 140.45 103.03) (width 0.2) (layer "F.Cu") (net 14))
 (segment (start 140.45 103.03) (end 139.96 102.54) (width 0.2) (layer "F.Cu") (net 14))
 (segment (start 139.96 102.54) (end 137.5 102.54) (width 0.2) (layer "F.Cu") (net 14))
 (via (at 140.45 104) (size 0.6) (drill 0.3) (layers "F.Cu" "B.Cu") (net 14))
 (segment (start 140.45 104) (end 140.5 104.05) (width 0.2) (layer "B.Cu") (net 14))
 (segment (start 140.5 105.42) (end 142.5 107.42) (width 0.2) (layer "B.Cu") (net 14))
 (segment (start 140.5 104.05) (end 140.5 105.42) (width 0.2) (layer "B.Cu") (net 14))
 (segment (start 146.4375 85.5) (end 146.875 85.9375) (width 0.2) (layer "F.Cu") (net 16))
 (segment (start 145.5 85.5) (end 146.4375 85.5) (width 0.2) (layer "F.Cu") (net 16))
 (segment (start 141.5 69.5) (end 141.48 69.52) (width 0.2) (layer "F.Cu") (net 16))
 (segment (start 144.5 84.5) (end 145.5 85.5) (width 0.2) (layer "F.Cu") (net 16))
 (segment (start 141 84.5) (end 144.5 84.5) (width 0.2) (layer "F.Cu") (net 16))
 (segment (start 144.5 85.86941) (end 142.36941 85.86941) (width 0.2) (layer "F.Cu") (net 16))
 (segment (start 141.54 115.04) (end 140 113.5) (width 0.2) (layer "F.Cu") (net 16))
 (segment (start 142.86 115.04) (end 141.54 115.04) (width 0.2) (layer "F.Cu") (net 16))
 (segment (start 144.5 85.86941) (end 145.50559 86.875) (width 0.2) (layer "F.Cu") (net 16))
 (segment (start 142.36941 85.86941) (end 141 84.5) (width 0.2) (layer "F.Cu") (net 16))
 (segment (start 145.50559 86.875) (end 145.9375 86.875) (width 0.2) (layer "F.Cu") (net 16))
 (segment (start 141.48 69.52) (end 137.5 69.52) (width 0.2) (layer "F.Cu") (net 16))
 (via (at 141.5 69.5) (size 0.6) (drill 0.3) (layers "F.Cu" "B.Cu") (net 16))
 (via (at 140 113.5) (size 0.6) (drill 0.3) (layers "F.Cu" "B.Cu") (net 16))
 (via (at 141 84.5) (size 0.6) (drill 0.3) (layers "F.Cu" "B.Cu") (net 16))
 (segment (start 142.5 73.5) (end 141 75) (width 0.2) (layer "B.Cu") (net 16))
 (segment (start 142.5 70.5) (end 142.5 73.5) (width 0.2) (layer "B.Cu") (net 16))
 (segment (start 141 86) (end 139.899 87.101) (width 0.2) (layer "B.Cu") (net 16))
 (segment (start 141 84.5) (end 141 86) (width 0.2) (layer "B.Cu") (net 16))
 (segment (start 142.5 70.5) (end 141.5 69.5) (width 0.2) (layer "B.Cu") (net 16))
 (segment (start 139.899 87.101) (end 139.899 113.399) (width 0.2) (layer "B.Cu") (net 16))
 (segment (start 141 75) (end 141 84.5) (width 0.2) (layer "B.Cu") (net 16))
 (segment (start 139.899 113.399) (end 140 113.5) (width 0.2) (layer "B.Cu") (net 16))
 (segment (start 141 67) (end 146 72) (width 0.2) (layer "F.Cu") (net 3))
 (segment (start 141 65) (end 141 67) (width 0.2) (layer "F.Cu") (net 3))
 (segment (start 150.43 71.75) (end 150.43 69.095) (width 0.2) (layer "F.Cu") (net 3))
 (segment (start 146 72) (end 150.18 72) (width 0.2) (layer "F.Cu") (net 3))
 (segment (start 150.18 72) (end 150.43 71.75) (width 0.2) (layer "F.Cu") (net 3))
 (segment (start 138 62) (end 128.62 62) (width 0.2) (layer "F.Cu") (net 3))
 (segment (start 126.81 63.81) (end 126.81 66.81) (width 0.2) (layer "F.Cu") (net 3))
 (segment (start 128.62 62) (end 126.81 63.81) (width 0.2) (layer "F.Cu") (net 3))
 (segment (start 138 62) (end 141 65) (width 0.2) (layer "F.Cu") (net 3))
 (segment (start 143.1 76.5) (end 141.5 76.5) (width 0.2) (layer "F.Cu") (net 1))
 (segment (start 147.5 83.5) (end 140 83.5) (width 0.2) (layer "F.Cu") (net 1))
 (segment (start 140 74.5) (end 140 75) (width 0.2) (layer "F.Cu") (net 1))
 (segment (start 147.375 85.9375) (end 147.375 85.5) (width 0.2) (layer "F.Cu") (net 1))
 (segment (start 145.509202 87.375) (end 145.9375 87.375) (width 0.2) (layer "F.Cu") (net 1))
 (segment (start 141.5 73) (end 140 74.5) (width 0.2) (layer "F.Cu") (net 1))
 (segment (start 140 83.5) (end 140 86) (width 0.2) (layer "F.Cu") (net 1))
 (segment (start 147.875 85.9375) (end 147.875 85) (width 0.2) (layer "F.Cu") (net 1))
 (segment (start 140 75) (end 141.5 76.5) (width 0.2) (layer "F.Cu") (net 1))
 (segment (start 145.134202 87) (end 145.509202 87.375) (width 0.2) (layer "F.Cu") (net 1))
 (segment (start 151 73) (end 141.5 73) (width 0.2) (layer "F.Cu") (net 1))
 (segment (start 147.875 83.875) (end 147.5 83.5) (width 0.2) (layer "F.Cu") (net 1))
 (segment (start 151.905 72.095) (end 151 73) (width 0.2) (layer "F.Cu") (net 1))
 (segment (start 147.875 85) (end 147.875 83.875) (width 0.2) (layer "F.Cu") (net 1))
 (segment (start 141.5 76.5) (end 140 78) (width 0.2) (layer "F.Cu") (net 1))
 (segment (start 140 78) (end 140 83.5) (width 0.2) (layer "F.Cu") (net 1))
 (segment (start 151.905 69.095) (end 151.905 72.095) (width 0.2) (layer "F.Cu") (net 1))
 (segment (start 141 87) (end 145.134202 87) (width 0.2) (layer "F.Cu") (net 1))
 (segment (start 140 86) (end 141 87) (width 0.2) (layer "F.Cu") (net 1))
 (segment (start 147.375 85.5) (end 147.875 85) (width 0.2) (layer "F.Cu") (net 1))
 (segment (start 151.555 87.875) (end 149.8125 87.875) (width 0.2) (layer "F.Cu") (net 17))
 (segment (start 143.375 88.865) (end 145.9275 88.865) (width 0.2) (layer "F.Cu") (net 5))
 (segment (start 145.9275 88.865) (end 145.9375 88.875) (width 0.2) (layer "F.Cu") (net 5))
 (segment (start 141 111.82) (end 139.34 110.16) (width 0.2) (layer "F.Cu") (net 4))
 (segment (start 151.375 88.875) (end 153 88.875) (width 0.2) (layer "F.Cu") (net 4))
 (segment (start 137.5 72.06) (end 141.44 72.06) (width 0.2) (layer "F.Cu") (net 4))
 (segment (start 145.9375 87.875) (end 144.765 87.875) (width 0.2) (layer "F.Cu") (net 4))
 (segment (start 149.88 70.735) (end 149.43 70.285) (width 0.2) (layer "F.Cu") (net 4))
 (segment (start 116 97.46) (end 118.12 97.46) (width 0.2) (layer "F.Cu") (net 4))
 (segment (start 153 88.875) (end 152.375 88.875) (width 0.2) (layer "F.Cu") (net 4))
 (segment (start 152.375 88.875) (end 152.195 88.695) (width 0.2) (layer "F.Cu") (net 4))
 (segment (start 139.34 110.16) (end 137.5 110.16) (width 0.2) (layer "F.Cu") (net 4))
 (segment (start 149.43 70.285) (end 149.43 69.095) (width 0.2) (layer "F.Cu") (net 4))
 (segment (start 141 112.5) (end 141 111.82) (width 0.2) (layer "F.Cu") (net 4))
 (segment (start 145.9375 88.375) (end 144.375 88.375) (width 0.2) (layer "F.Cu") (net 4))
 (segment (start 141.44 72.06) (end 141.5 72) (width 0.2) (layer "F.Cu") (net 4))
 (segment (start 115.5 84.76) (end 118.12 84.76) (width 0.2) (layer "F.Cu") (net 4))
 (segment (start 148.875 88.875) (end 149.8125 88.875) (width 0.2) (layer "F.Cu") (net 4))
 (segment (start 147.875 87.875) (end 148.875 88.875) (width 0.2) (layer "F.Cu") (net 4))
 (segment (start 145 76.5) (end 146.6 76.5) (width 0.2) (layer "F.Cu") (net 4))
 (segment (start 140.46 97.46) (end 140.5 97.5) (width 0.2) (layer "F.Cu") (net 4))
 (segment (start 147.628612 82.95) (end 146 82.95) (width 0.2) (layer "F.Cu") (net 4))
 (segment (start 149.8125 88.875) (end 151.375 88.875) (width 0.2) (layer "F.Cu") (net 4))
 (segment (start 148.375 83.696388) (end 147.628612 82.95) (width 0.2) (layer "F.Cu") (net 4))
 (segment (start 150.5175 76.9675) (end 148.5325 76.9675) (width 0.2) (layer "F.Cu") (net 4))
 (segment (start 137.5 97.46) (end 140.46 97.46) (width 0.2) (layer "F.Cu") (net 4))
 (segment (start 148.375 85.9375) (end 148.375 83.696388) (width 0.2) (layer "F.Cu") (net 4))
 (segment (start 149.43 69.095) (end 149.43 70.235) (width 0.2) (layer "F.Cu") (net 4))
 (segment (start 149.8125 88.375) (end 150.875 88.375) (width 0.2) (layer "F.Cu") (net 4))
 (segment (start 115.5 72) (end 115.56 72.06) (width 0.2) (layer "F.Cu") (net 4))
 (segment (start 149.88 70.735) (end 149.93 70.685) (width 0.2) (layer "F.Cu") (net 4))
 (segment (start 145.125 80.5) (end 146.675 80.5) (width 0.2) (layer "F.Cu") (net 4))
 (segment (start 148.875 89.8125) (end 148.875 91.375) (width 0.2) (layer "F.Cu") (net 4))
 (segment (start 148.375 89.8125) (end 148.375 91.875) (width 0.2) (layer "F.Cu") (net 4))
 (segment (start 149.93 70.685) (end 149.93 69.095) (width 0.2) (layer "F.Cu") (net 4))
 (segment (start 152.195 88.695) (end 152.195 87.875) (width 0.2) (layer "F.Cu") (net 4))
 (segment (start 115.56 72.06) (end 118.12 72.06) (width 0.2) (layer "F.Cu") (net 4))
 (segment (start 144.765 87.875) (end 144.375 88.265) (width 0.2) (layer "F.Cu") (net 4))
 (segment (start 115.66 110.16) (end 118.12 110.16) (width 0.2) (layer "F.Cu") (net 4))
 (segment (start 130.9341 98.9341) (end 131 99) (width 0.2) (layer "F.Cu") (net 4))
 (segment (start 130.9341 96.81) (end 130.9341 98.9341) (width 0.2) (layer "F.Cu") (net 4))
 (segment (start 150.875 88.375) (end 151.375 88.875) (width 0.2) (layer "F.Cu") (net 4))
 (segment (start 143.375 89.885) (end 143.375 90.875) (width 0.2) (layer "F.Cu") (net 4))
 (segment (start 141 112.5) (end 142.5 112.5) (width 0.2) (layer "F.Cu") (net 4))
 (segment (start 148.5325 76.9675) (end 148.5 77) (width 0.2) (layer "F.Cu") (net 4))
 (segment (start 144.375 88.375) (end 144.375 88.265) (width 0.2) (layer "F.Cu") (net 4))
 (segment (start 148.875 91.375) (end 148.375 91.875) (width 0.2) (layer "F.Cu") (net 4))
 (via (at 148.375 91.875) (size 0.6) (drill 0.3) (layers "F.Cu" "B.Cu") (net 4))
 (via (at 115.5 84.76) (size 0.6) (drill 0.3) (layers "F.Cu" "B.Cu") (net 4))
 (via (at 115.66 110.16) (size 0.6) (drill 0.3) (layers "F.Cu" "B.Cu") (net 4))
 (via (at 131 99) (size 0.6) (drill 0.3) (layers "F.Cu" "B.Cu") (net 4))
 (via (at 153 88.875) (size 0.6) (drill 0.3) (layers "F.Cu" "B.Cu") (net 4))
 (via (at 141 112.5) (size 0.6) (drill 0.3) (layers "F.Cu" "B.Cu") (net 4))
 (via (at 146.6 76.5) (size 0.6) (drill 0.3) (layers "F.Cu" "B.Cu") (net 4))
 (via (at 140.5 97.5) (size 0.6) (drill 0.3) (layers "F.Cu" "B.Cu") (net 4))
 (via (at 144.375 88.265) (size 0.6) (drill 0.3) (layers "F.Cu" "B.Cu") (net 4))
 (via (at 149.88 70.735) (size 0.6) (drill 0.3) (layers "F.Cu" "B.Cu") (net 4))
 (via (at 116 97.46) (size 0.6) (drill 0.3) (layers "F.Cu" "B.Cu") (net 4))
 (via (at 146.675 80.5) (size 0.6) (drill 0.3) (layers "F.Cu" "B.Cu") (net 4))
 (via (at 141.5 72) (size 0.6) (drill 0.3) (layers "F.Cu" "B.Cu") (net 4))
 (via (at 143.375 90.875) (size 0.6) (drill 0.3) (layers "F.Cu" "B.Cu") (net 4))
 (via (at 148.5 77) (size 0.6) (drill 0.3) (layers "F.Cu" "B.Cu") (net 4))
 (via (at 115.5 72) (size 0.6) (drill 0.3) (layers "F.Cu" "B.Cu") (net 4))
 (via (at 146 82.95) (size 0.6) (drill 0.3) (layers "F.Cu" "B.Cu") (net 4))
 (segment (start 142.5 109.96) (end 141 108.46) (width 0.2) (layer "F.Cu") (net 15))
 (segment (start 141 108.46) (end 141 101.5) (width 0.2) (layer "F.Cu") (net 15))
 (segment (start 141 101.5) (end 139.5 100) (width 0.2) (layer "F.Cu") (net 15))
 (segment (start 139.5 100) (end 137.5 100) (width 0.2) (layer "F.Cu") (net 15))
 (segment (start 150.875 86.875) (end 150.875 85.8125) (width 0.2) (layer "F.Cu") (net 18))
 (segment (start 148.875 83.7) (end 149.3375 84.1625) (width 0.2) (layer "F.Cu") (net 18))
 (segment (start 150.5175 78.9675) (end 148.5325 78.9675) (width 0.2) (layer "F.Cu") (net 18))
 (segment (start 150.3375 85.1625) (end 150.875 85.7) (width 0.2) (layer "F.Cu") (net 18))
 (segment (start 147.574 82.399) (end 144.101 82.399) (width 0.2) (layer "F.Cu") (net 18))
 (segment (start 148.5325 78.9675) (end 147.5875 79.9125) (width 0.2) (layer "F.Cu") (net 18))
 (segment (start 149.3375 84.1625) (end 150.3375 85.1625) (width 0.2) (layer "F.Cu") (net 18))
 (segment (start 149.8125 86.875) (end 150.875 85.8125) (width 0.2) (layer "F.Cu") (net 18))
 (segment (start 150.375 87.375) (end 150.875 86.875) (width 0.2) (layer "F.Cu") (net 18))
 (segment (start 148.875 83.7) (end 147.5875 82.4125) (width 0.2) (layer "F.Cu") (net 18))
 (segment (start 147.5875 79.9125) (end 147.5875 82.4125) (width 0.2) (layer "F.Cu") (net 18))
 (segment (start 149.8125 87.375) (end 150.375 87.375) (width 0.2) (layer "F.Cu") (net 18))
 (segment (start 150.875 85.7) (end 150.875 85.8125) (width 0.2) (layer "F.Cu") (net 18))
 (segment (start 144.101 82.399) (end 144 82.5) (width 0.2) (layer "F.Cu") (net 18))
 (segment (start 144 82.5) (end 143.225 81.725) (width 0.2) (layer "F.Cu") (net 18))
 (segment (start 148.875 85.9375) (end 148.875 83.7) (width 0.2) (layer "F.Cu") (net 18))
 (segment (start 147.5875 82.4125) (end 147.574 82.399) (width 0.2) (layer "F.Cu") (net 18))
 (segment (start 143.225 81.725) (end 143.225 80.5) (width 0.2) (layer "F.Cu") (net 18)))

